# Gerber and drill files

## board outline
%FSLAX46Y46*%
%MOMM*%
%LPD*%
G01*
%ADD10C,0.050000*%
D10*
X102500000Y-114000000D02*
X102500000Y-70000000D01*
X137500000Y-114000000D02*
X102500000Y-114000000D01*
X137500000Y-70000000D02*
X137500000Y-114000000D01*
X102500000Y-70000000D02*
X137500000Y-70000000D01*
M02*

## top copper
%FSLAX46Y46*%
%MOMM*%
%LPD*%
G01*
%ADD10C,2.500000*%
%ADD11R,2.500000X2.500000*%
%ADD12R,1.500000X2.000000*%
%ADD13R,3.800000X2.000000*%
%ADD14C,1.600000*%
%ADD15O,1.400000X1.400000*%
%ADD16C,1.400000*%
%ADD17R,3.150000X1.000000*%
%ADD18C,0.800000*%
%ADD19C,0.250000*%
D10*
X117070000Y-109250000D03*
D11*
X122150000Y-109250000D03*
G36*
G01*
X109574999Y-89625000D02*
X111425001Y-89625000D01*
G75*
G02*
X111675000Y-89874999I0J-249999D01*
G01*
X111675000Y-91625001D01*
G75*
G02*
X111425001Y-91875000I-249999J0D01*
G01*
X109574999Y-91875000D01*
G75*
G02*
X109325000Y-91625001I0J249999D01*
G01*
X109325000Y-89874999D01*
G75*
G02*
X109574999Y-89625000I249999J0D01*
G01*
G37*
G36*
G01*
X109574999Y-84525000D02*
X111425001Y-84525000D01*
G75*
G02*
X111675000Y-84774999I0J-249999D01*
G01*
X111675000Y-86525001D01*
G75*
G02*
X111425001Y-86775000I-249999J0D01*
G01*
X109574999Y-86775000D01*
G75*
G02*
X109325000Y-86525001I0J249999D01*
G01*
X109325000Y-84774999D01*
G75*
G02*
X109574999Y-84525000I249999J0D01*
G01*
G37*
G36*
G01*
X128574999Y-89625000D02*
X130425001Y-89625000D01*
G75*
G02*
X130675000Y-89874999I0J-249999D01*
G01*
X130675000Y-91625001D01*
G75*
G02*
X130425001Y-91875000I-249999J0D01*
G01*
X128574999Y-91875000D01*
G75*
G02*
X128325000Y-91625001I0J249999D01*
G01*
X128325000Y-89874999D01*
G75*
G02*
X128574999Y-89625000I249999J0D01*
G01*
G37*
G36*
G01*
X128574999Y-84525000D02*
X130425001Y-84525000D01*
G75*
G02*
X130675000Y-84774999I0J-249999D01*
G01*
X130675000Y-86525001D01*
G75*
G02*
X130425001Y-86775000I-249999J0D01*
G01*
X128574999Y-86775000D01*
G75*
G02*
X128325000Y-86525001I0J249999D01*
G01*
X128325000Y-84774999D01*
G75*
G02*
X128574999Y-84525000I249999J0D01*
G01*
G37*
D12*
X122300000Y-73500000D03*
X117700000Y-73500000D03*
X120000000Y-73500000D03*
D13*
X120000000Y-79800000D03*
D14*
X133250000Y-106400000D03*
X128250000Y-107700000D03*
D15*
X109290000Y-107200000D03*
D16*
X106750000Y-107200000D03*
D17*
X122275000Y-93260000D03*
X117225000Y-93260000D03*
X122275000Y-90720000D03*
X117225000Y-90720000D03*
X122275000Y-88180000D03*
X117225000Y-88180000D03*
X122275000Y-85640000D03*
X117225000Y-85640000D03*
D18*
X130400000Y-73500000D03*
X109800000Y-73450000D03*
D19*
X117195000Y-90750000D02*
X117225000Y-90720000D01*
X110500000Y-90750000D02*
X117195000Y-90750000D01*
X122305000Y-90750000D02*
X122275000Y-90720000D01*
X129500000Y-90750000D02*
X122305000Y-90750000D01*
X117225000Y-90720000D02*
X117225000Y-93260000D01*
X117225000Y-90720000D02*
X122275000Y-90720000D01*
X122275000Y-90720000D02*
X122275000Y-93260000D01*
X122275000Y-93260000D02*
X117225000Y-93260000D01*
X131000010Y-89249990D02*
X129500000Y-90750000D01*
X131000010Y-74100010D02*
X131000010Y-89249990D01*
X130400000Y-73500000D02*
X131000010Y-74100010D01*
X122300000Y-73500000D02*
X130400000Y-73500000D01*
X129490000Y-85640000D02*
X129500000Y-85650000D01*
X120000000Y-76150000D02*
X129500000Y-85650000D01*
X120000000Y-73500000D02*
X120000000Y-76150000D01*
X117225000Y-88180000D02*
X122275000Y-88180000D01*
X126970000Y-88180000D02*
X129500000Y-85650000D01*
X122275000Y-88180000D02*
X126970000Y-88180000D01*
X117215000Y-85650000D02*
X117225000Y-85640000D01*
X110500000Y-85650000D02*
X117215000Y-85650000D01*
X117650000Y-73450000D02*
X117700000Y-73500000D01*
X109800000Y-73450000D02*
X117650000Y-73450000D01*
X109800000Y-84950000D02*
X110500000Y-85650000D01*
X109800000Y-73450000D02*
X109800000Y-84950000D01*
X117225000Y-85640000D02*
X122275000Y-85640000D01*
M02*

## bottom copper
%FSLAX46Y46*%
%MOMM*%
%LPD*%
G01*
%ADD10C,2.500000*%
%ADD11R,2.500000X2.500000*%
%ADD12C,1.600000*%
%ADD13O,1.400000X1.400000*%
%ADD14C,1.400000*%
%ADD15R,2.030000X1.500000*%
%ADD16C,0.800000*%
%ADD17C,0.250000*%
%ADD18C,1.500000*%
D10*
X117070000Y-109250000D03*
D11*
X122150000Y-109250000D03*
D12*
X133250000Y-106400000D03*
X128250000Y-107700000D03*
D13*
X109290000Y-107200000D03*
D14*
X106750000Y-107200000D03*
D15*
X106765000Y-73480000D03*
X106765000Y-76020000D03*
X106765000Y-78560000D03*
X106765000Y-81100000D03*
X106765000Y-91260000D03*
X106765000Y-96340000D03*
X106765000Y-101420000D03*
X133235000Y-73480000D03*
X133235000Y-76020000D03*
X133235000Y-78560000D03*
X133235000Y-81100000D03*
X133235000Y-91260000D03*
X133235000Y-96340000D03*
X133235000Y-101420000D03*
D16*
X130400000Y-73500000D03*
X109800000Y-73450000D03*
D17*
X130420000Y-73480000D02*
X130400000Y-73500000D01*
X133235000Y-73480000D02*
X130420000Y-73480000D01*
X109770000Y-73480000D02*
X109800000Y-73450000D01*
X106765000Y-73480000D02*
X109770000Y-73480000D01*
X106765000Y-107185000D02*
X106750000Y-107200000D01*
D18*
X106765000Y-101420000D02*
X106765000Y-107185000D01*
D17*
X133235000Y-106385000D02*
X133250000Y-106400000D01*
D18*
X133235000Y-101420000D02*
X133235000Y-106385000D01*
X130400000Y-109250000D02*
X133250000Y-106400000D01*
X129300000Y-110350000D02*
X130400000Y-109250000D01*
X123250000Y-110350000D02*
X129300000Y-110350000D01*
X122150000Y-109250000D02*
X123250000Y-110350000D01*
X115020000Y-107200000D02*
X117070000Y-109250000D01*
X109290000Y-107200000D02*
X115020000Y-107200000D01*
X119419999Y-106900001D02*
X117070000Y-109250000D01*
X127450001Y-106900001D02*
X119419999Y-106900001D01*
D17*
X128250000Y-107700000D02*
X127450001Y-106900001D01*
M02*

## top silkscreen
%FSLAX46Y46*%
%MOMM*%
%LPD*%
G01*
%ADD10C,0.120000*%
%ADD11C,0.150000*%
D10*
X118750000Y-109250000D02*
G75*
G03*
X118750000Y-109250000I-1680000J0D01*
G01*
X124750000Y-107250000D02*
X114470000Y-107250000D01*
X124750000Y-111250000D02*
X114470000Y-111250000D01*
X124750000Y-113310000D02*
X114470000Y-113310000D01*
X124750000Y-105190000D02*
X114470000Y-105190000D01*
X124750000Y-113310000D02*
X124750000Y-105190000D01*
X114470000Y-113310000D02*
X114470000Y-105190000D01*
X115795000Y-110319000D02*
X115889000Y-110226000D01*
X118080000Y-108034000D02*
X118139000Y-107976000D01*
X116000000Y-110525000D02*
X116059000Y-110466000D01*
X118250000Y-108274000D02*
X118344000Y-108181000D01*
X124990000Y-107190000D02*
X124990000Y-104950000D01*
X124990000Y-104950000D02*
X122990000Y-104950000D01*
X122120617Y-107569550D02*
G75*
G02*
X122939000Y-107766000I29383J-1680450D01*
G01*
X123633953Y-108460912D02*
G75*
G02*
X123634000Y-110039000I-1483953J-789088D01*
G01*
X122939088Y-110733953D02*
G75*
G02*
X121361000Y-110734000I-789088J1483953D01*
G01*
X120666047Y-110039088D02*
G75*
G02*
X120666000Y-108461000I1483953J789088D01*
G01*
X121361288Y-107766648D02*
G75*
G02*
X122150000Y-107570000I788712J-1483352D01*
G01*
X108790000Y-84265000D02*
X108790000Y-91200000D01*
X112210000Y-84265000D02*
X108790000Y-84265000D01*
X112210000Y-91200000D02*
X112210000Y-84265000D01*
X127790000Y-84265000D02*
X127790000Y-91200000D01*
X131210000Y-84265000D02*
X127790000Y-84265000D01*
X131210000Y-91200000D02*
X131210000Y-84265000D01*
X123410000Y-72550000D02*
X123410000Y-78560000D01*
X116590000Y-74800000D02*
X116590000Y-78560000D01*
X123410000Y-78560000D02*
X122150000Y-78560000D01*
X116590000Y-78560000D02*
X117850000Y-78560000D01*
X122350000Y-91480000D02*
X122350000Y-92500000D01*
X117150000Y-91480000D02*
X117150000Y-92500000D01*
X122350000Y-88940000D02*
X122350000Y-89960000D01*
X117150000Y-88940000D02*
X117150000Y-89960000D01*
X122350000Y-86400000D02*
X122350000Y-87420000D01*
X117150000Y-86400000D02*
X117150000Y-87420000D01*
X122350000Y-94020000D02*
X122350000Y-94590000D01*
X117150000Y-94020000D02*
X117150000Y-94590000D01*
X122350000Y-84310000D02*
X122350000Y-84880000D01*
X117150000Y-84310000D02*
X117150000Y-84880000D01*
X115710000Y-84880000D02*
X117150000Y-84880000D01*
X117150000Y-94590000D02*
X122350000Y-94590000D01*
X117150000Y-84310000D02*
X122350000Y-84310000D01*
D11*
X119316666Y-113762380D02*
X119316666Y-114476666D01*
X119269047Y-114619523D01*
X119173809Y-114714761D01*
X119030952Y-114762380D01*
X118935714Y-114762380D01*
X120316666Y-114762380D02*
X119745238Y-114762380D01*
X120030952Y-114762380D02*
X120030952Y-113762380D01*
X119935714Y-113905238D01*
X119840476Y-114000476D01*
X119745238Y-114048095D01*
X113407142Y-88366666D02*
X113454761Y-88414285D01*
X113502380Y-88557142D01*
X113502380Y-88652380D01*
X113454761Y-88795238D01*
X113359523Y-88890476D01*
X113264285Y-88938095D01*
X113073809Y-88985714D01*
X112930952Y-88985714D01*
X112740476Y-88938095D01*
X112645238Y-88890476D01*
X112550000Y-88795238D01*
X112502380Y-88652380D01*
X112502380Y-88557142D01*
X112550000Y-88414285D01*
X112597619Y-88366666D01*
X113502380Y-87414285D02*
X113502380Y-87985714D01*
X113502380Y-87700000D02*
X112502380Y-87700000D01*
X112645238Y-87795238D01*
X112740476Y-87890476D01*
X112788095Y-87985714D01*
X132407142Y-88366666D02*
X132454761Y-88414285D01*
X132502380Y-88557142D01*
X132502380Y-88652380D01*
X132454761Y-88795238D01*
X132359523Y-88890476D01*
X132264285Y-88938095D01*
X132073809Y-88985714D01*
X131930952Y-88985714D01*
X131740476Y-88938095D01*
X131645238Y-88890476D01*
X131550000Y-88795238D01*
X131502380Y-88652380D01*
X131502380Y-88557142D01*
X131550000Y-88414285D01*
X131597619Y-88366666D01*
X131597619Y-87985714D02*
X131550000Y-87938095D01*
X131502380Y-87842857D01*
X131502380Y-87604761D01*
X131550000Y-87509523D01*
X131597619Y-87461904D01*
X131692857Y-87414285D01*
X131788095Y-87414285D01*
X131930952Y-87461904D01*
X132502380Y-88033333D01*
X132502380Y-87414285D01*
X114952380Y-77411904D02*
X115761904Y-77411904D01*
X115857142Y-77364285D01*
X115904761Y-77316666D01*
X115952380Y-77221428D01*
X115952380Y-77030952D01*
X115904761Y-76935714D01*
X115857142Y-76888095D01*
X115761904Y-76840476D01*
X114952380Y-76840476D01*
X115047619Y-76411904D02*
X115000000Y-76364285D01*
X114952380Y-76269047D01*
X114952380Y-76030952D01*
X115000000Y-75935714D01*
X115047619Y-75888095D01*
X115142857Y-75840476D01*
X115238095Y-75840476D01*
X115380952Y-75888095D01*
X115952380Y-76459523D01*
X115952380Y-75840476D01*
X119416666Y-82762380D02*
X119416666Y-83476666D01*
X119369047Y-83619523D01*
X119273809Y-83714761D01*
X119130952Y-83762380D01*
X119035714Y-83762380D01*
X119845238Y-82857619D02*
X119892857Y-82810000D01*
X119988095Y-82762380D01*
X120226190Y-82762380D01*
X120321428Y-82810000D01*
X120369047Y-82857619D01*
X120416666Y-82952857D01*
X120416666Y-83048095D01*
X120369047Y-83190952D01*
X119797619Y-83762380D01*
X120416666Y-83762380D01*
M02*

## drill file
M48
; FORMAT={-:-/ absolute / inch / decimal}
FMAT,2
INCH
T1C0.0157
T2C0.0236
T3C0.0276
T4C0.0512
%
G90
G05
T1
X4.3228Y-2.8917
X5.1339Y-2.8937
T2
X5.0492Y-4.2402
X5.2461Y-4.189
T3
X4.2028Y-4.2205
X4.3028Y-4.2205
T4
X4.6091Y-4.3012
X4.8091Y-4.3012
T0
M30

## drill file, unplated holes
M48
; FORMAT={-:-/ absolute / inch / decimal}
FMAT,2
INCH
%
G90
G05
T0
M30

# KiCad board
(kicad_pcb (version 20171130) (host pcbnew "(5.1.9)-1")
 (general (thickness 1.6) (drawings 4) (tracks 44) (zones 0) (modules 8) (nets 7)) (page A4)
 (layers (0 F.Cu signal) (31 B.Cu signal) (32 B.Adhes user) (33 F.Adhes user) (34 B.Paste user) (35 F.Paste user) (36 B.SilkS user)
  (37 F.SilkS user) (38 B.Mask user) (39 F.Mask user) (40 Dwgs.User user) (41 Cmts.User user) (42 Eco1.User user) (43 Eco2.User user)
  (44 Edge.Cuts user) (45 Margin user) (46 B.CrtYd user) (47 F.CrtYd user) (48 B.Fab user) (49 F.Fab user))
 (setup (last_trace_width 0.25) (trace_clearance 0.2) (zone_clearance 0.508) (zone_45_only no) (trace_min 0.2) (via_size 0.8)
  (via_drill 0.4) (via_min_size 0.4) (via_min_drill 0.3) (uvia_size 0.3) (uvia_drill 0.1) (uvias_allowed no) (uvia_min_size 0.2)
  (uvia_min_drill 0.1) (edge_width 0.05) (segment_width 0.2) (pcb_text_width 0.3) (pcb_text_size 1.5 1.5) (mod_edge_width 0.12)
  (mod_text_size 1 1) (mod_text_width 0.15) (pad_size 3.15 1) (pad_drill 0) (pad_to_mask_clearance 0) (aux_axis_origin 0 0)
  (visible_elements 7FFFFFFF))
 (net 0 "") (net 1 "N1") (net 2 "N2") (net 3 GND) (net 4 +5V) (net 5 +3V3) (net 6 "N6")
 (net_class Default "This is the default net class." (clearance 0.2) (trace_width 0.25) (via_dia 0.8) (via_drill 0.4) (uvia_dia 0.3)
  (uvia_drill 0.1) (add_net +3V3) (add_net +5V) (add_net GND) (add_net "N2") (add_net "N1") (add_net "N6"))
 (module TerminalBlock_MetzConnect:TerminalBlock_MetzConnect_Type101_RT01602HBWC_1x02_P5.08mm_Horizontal (layer F.Cu) (at 122.15 109.25 180)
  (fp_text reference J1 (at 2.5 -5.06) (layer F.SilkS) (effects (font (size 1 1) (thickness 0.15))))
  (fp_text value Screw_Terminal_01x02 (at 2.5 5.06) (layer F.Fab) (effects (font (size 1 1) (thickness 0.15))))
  (fp_circle (center 5.08 0) (end 6.76 0) (layer F.SilkS) (width 0.12))
  (fp_line (start -2.6 2) (end 7.68 2) (layer F.SilkS) (width 0.12))
  (fp_line (start -2.6 -2) (end 7.68 -2) (layer F.SilkS) (width 0.12))
  (fp_line (start -2.6 -4.06) (end 7.68 -4.06) (layer F.SilkS) (width 0.12))
  (fp_line (start -2.6 4.06) (end 7.68 4.06) (layer F.SilkS) (width 0.12))
  (fp_line (start -2.6 -4.06) (end -2.6 4.06) (layer F.SilkS) (width 0.12))
  (fp_line (start 7.68 -4.06) (end 7.68 4.06) (layer F.SilkS) (width 0.12))
  (fp_line (start 6.355 -1.069) (end 6.261 -0.976) (layer F.SilkS) (width 0.12))
  (fp_line (start 4.07 1.216) (end 4.011 1.274) (layer F.SilkS) (width 0.12))
  (fp_line (start 6.15 -1.275) (end 6.091 -1.216) (layer F.SilkS) (width 0.12))
  (fp_line (start 3.9 0.976) (end 3.806 1.069) (layer F.SilkS) (width 0.12))
  (fp_line (start -2.84 2.06) (end -2.84 4.3) (layer F.SilkS) (width 0.12))
  (fp_line (start -2.84 4.3) (end -0.84 4.3) (layer F.SilkS) (width 0.12))
  (fp_arc (start 0 0) (end -0.789 1.484) (angle -29) (layer F.SilkS) (width 0.12))
  (fp_arc (start 0 0) (end -1.484 -0.789) (angle -56) (layer F.SilkS) (width 0.12))
  (fp_arc (start 0 0) (end 0.789 -1.484) (angle -56) (layer F.SilkS) (width 0.12))
  (fp_arc (start 0 0) (end 1.484 0.789) (angle -56) (layer F.SilkS) (width 0.12))
  (fp_arc (start 0 0) (end 0 1.68) (angle -28) (layer F.SilkS) (width 0.12))
  (pad 2 thru_hole circle (at 5.08 0 180) (size 2.5 2.5) (drill 1.3) (layers *.Cu *.Mask) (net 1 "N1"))
  (pad 1 thru_hole rect (at 0 0 180) (size 2.5 2.5) (drill 1.3) (layers *.Cu *.Mask) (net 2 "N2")))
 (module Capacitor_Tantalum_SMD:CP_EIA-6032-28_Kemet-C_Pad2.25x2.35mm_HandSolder (layer F.Cu) (at 110.5 88.2 270)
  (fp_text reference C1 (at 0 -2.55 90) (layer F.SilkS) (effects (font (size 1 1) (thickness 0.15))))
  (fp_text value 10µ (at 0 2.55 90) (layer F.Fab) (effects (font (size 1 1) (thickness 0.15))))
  (fp_line (start -3.935 1.71) (end 3 1.71) (layer F.SilkS) (width 0.12))
  (fp_line (start -3.935 -1.71) (end -3.935 1.71) (layer F.SilkS) (width 0.12))
  (fp_line (start 3 -1.71) (end -3.935 -1.71) (layer F.SilkS) (width 0.12))
  (pad 2 smd roundrect (at 2.55 0 270) (size 2.25 2.35) (layers F.Cu F.Paste F.Mask) (roundrect_rratio 0.1111106666666667) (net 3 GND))
  (pad 1 smd roundrect (at -2.55 0 270) (size 2.25 2.35) (layers F.Cu F.Paste F.Mask) (roundrect_rratio 0.1111106666666667) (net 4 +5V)))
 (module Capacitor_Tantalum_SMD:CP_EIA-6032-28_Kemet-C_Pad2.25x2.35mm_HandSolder (layer F.Cu) (at 129.5 88.2 270)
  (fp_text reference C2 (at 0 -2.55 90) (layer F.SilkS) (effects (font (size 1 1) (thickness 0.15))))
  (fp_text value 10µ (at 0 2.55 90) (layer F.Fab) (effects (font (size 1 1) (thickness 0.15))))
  (fp_line (start -3.935 1.71) (end 3 1.71) (layer F.SilkS) (width 0.12))
  (fp_line (start -3.935 -1.71) (end -3.935 1.71) (layer F.SilkS) (width 0.12))
  (fp_line (start 3 -1.71) (end -3.935 -1.71) (layer F.SilkS) (width 0.12))
  (pad 2 smd roundrect (at 2.55 0 270) (size 2.25 2.35) (layers F.Cu F.Paste F.Mask) (roundrect_rratio 0.1111106666666667) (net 3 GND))
  (pad 1 smd roundrect (at -2.55 0 270) (size 2.25 2.35) (layers F.Cu F.Paste F.Mask) (roundrect_rratio 0.1111106666666667) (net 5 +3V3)))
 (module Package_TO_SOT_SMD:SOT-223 (layer F.Cu) (at 120 76.65 270)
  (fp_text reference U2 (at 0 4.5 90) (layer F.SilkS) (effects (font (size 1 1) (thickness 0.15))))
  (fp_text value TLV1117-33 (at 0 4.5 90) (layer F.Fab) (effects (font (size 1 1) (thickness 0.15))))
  (fp_line (start -4.1 -3.41) (end 1.91 -3.41) (layer F.SilkS) (width 0.12))
  (fp_line (start -1.85 3.41) (end 1.91 3.41) (layer F.SilkS) (width 0.12))
  (fp_line (start 1.91 -3.41) (end 1.91 -2.15) (layer F.SilkS) (width 0.12))
  (fp_line (start 1.91 3.41) (end 1.91 2.15) (layer F.SilkS) (width 0.12))
  (pad 1 smd rect (at -3.15 -2.3 270) (size 2 1.5) (layers F.Cu F.Paste F.Mask) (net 3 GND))
  (pad 3 smd rect (at -3.15 2.3 270) (size 2 1.5) (layers F.Cu F.Paste F.Mask) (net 4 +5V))
  (pad 2 smd rect (at -3.15 0 270) (size 2 1.5) (layers F.Cu F.Paste F.Mask) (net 5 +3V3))
  (pad 4 smd rect (at 3.15 0 270) (size 2 3.8) (layers F.Cu F.Paste F.Mask)))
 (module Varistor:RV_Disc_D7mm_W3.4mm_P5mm (layer B.Cu) (at 128.25 107.7)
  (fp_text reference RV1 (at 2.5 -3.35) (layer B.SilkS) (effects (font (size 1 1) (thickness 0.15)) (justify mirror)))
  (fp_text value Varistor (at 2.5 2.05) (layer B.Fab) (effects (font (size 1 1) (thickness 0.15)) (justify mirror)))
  (pad 2 thru_hole circle (at 5 -1.3) (size 1.6 1.6) (drill 0.6) (layers *.Cu *.Mask) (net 2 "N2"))
  (pad 1 thru_hole circle (at 0 0) (size 1.6 1.6) (drill 0.6) (layers *.Cu *.Mask) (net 1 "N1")))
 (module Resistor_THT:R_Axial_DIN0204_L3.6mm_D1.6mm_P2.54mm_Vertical (layer B.Cu) (at 106.75 107.2)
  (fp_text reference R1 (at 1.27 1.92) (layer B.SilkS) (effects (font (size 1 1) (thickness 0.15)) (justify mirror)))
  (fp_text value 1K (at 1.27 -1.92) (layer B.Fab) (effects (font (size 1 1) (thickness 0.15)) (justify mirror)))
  (pad 2 thru_hole oval (at 2.54 0) (size 1.4 1.4) (drill 0.7) (layers *.Cu *.Mask) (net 1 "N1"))
  (pad 1 thru_hole circle (at 0 0) (size 1.4 1.4) (drill 0.7) (layers *.Cu *.Mask) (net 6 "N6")))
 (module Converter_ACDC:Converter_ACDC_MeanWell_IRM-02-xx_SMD (layer B.Cu) (at 120 87.45)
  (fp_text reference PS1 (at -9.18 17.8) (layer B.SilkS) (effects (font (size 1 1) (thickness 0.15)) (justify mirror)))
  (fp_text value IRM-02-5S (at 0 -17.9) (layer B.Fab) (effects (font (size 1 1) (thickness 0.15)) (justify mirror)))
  (pad 12 smd rect (at -13.235 -13.97 90) (size 1.5 2.03) (layers B.Cu B.Paste B.Mask) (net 4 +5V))
  (pad 11 smd rect (at -13.235 -11.43 90) (size 1.5 2.03) (layers B.Cu B.Paste B.Mask))
  (pad 10 smd rect (at -13.235 -8.89 90) (size 1.5 2.03) (layers B.Cu B.Paste B.Mask))
  (pad 9 smd rect (at -13.235 -6.35 90) (size 1.5 2.03) (layers B.Cu B.Paste B.Mask))
  (pad 5 smd rect (at -13.235 3.81 90) (size 1.5 2.03) (layers B.Cu B.Paste B.Mask))
  (pad 3 smd rect (at -13.235 8.89 90) (size 1.5 2.03) (layers B.Cu B.Paste B.Mask))
  (pad 1 smd rect (at -13.235 13.97 90) (size 1.5 2.03) (layers B.Cu B.Paste B.Mask) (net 6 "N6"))
  (pad 13 smd rect (at 13.235 -13.97 90) (size 1.5 2.03) (layers B.Cu B.Paste B.Mask) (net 3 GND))
  (pad 14 smd rect (at 13.235 -11.43 90) (size 1.5 2.03) (layers B.Cu B.Paste B.Mask))
  (pad 15 smd rect (at 13.235 -8.89 90) (size 1.5 2.03) (layers B.Cu B.Paste B.Mask))
  (pad 16 smd rect (at 13.235 -6.35 90) (size 1.5 2.03) (layers B.Cu B.Paste B.Mask))
  (pad 20 smd rect (at 13.235 3.81 90) (size 1.5 2.03) (layers B.Cu B.Paste B.Mask))
  (pad 22 smd rect (at 13.235 8.89 90) (size 1.5 2.03) (layers B.Cu B.Paste B.Mask))
  (pad 24 smd rect (at 13.235 13.97 90) (size 1.5 2.03) (layers B.Cu B.Paste B.Mask) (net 2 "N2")))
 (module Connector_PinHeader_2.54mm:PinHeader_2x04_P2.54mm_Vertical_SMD (layer F.Cu) (at 119.75 89.45)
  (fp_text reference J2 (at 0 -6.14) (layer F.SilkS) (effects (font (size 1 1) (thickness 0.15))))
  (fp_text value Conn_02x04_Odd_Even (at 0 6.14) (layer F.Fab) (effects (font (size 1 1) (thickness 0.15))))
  (fp_line (start 2.6 2.03) (end 2.6 3.05) (layer F.SilkS) (width 0.12))
  (fp_line (start -2.6 2.03) (end -2.6 3.05) (layer F.SilkS) (width 0.12))
  (fp_line (start 2.6 -0.51) (end 2.6 0.51) (layer F.SilkS) (width 0.12))
  (fp_line (start -2.6 -0.51) (end -2.6 0.51) (layer F.SilkS) (width 0.12))
  (fp_line (start 2.6 -3.05) (end 2.6 -2.03) (layer F.SilkS) (width 0.12))
  (fp_line (start -2.6 -3.05) (end -2.6 -2.03) (layer F.SilkS) (width 0.12))
  (fp_line (start 2.6 4.57) (end 2.6 5.14) (layer F.SilkS) (width 0.12))
  (fp_line (start -2.6 4.57) (end -2.6 5.14) (layer F.SilkS) (width 0.12))
  (fp_line (start 2.6 -5.14) (end 2.6 -4.57) (layer F.SilkS) (width 0.12))
  (fp_line (start -2.6 -5.14) (end -2.6 -4.57) (layer F.SilkS) (width 0.12))
  (fp_line (start -4.04 -4.57) (end -2.6 -4.57) (layer F.SilkS) (width 0.12))
  (fp_line (start -2.6 5.14) (end 2.6 5.14) (layer F.SilkS) (width 0.12))
  (fp_line (start -2.6 -5.14) (end 2.6 -5.14) (layer F.SilkS) (width 0.12))
  (pad 8 smd rect (at 2.525 3.81) (size 3.15 1) (layers F.Cu F.Paste F.Mask) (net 3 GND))
  (pad 7 smd rect (at -2.525 3.81) (size 3.15 1) (layers F.Cu F.Paste F.Mask) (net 3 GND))
  (pad 6 smd rect (at 2.525 1.27) (size 3.15 1) (layers F.Cu F.Paste F.Mask) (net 3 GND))
  (pad 5 smd rect (at -2.525 1.27) (size 3.15 1) (layers F.Cu F.Paste F.Mask) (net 3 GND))
  (pad 4 smd rect (at 2.525 -1.27) (size 3.15 1) (layers F.Cu F.Paste F.Mask) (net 5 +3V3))
  (pad 3 smd rect (at -2.525 -1.27) (size 3.15 1) (layers F.Cu F.Paste F.Mask) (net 5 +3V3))
  (pad 2 smd rect (at 2.525 -3.81) (size 3.15 1) (layers F.Cu F.Paste F.Mask) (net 4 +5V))
  (pad 1 smd rect (at -2.525 -3.81) (size 3.15 1) (layers F.Cu F.Paste F.Mask) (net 4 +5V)))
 (gr_line (start 102.5 114) (end 102.5 70) (layer Edge.Cuts) (width 0.05))
 (gr_line (start 137.5 114) (end 102.5 114) (layer Edge.Cuts) (width 0.05))
 (gr_line (start 137.5 70) (end 137.5 114) (layer Edge.Cuts) (width 0.05))
 (gr_line (start 102.5 70) (end 137.5 70) (layer Edge.Cuts) (width 0.05))
 (via (at 130.4 73.5) (size 0.8) (drill 0.4) (layers F.Cu B.Cu) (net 3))
 (segment (start 117.195 90.75) (end 117.225 90.72) (width 0.25) (layer F.Cu) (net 3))
 (segment (start 110.5 90.75) (end 117.195 90.75) (width 0.25) (layer F.Cu) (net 3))
 (segment (start 122.305 90.75) (end 122.275 90.72) (width 0.25) (layer F.Cu) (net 3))
 (segment (start 129.5 90.75) (end 122.305 90.75) (width 0.25) (layer F.Cu) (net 3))
 (segment (start 117.225 90.72) (end 117.225 93.26) (width 0.25) (layer F.Cu) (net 3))
 (segment (start 117.225 90.72) (end 122.275 90.72) (width 0.25) (layer F.Cu) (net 3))
 (segment (start 122.275 90.72) (end 122.275 93.26) (width 0.25) (layer F.Cu) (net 3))
 (segment (start 122.275 93.26) (end 117.225 93.26) (width 0.25) (layer F.Cu) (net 3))
 (segment (start 130.42 73.48) (end 130.4 73.5) (width 0.25) (layer B.Cu) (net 3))
 (segment (start 133.235 73.48) (end 130.42 73.48) (width 0.25) (layer B.Cu) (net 3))
 (segment (start 131.00001 89.24999) (end 129.5 90.75) (width 0.25) (layer F.Cu) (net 3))
 (segment (start 131.00001 74.10001) (end 131.00001 89.24999) (width 0.25) (layer F.Cu) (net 3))
 (segment (start 130.4 73.5) (end 131.00001 74.10001) (width 0.25) (layer F.Cu) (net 3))
 (segment (start 122.3 73.5) (end 130.4 73.5) (width 0.25) (layer F.Cu) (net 3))
 (segment (start 129.49 85.64) (end 129.5 85.65) (width 0.25) (layer F.Cu) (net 5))
 (segment (start 120 76.15) (end 129.5 85.65) (width 0.25) (layer F.Cu) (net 5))
 (segment (start 120 73.5) (end 120 76.15) (width 0.25) (layer F.Cu) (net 5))
 (segment (start 117.225 88.18) (end 122.275 88.18) (width 0.25) (layer F.Cu) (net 5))
 (segment (start 126.97 88.18) (end 129.5 85.65) (width 0.25) (layer F.Cu) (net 5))
 (segment (start 122.275 88.18) (end 126.97 88.18) (width 0.25) (layer F.Cu) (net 5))
 (via (at 109.8 73.45) (size 0.8) (drill 0.4) (layers F.Cu B.Cu) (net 4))
 (segment (start 117.215 85.65) (end 117.225 85.64) (width 0.25) (layer F.Cu) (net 4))
 (segment (start 110.5 85.65) (end 117.215 85.65) (width 0.25) (layer F.Cu) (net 4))
 (segment (start 109.77 73.48) (end 109.8 73.45) (width 0.25) (layer B.Cu) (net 4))
 (segment (start 106.765 73.48) (end 109.77 73.48) (width 0.25) (layer B.Cu) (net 4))
 (segment (start 117.65 73.45) (end 117.7 73.5) (width 0.25) (layer F.Cu) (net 4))
 (segment (start 109.8 73.45) (end 117.65 73.45) (width 0.25) (layer F.Cu) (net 4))
 (segment (start 109.8 84.95) (end 110.5 85.65) (width 0.25) (layer F.Cu) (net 4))
 (segment (start 109.8 73.45) (end 109.8 84.95) (width 0.25) (layer F.Cu) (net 4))
 (segment (start 117.225 85.64) (end 122.275 85.64) (width 0.25) (layer F.Cu) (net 4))
 (segment (start 106.765 107.185) (end 106.75 107.2) (width 0.25) (layer B.Cu) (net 6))
 (segment (start 106.765 101.42) (end 106.765 107.185) (width 1.5) (layer B.Cu) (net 6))
 (segment (start 133.235 106.385) (end 133.25 106.4) (width 0.25) (layer B.Cu) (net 2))
 (segment (start 133.235 101.42) (end 133.235 106.385) (width 1.5) (layer B.Cu) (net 2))
 (segment (start 130.4 109.25) (end 133.25 106.4) (width 1.5) (layer B.Cu) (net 2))
 (segment (start 129.3 110.35) (end 130.4 109.25) (width 1.5) (layer B.Cu) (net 2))
 (segment (start 123.25 110.35) (end 129.3 110.35) (width 1.5) (layer B.Cu) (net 2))
 (segment (start 122.15 109.25) (end 123.25 110.35) (width 1.5) (layer B.Cu) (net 2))
 (segment (start 115.02 107.2) (end 117.07 109.25) (width 1.5) (layer B.Cu) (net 1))
 (segment (start 109.29 107.2) (end 115.02 107.2) (width 1.5) (layer B.Cu) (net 1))
 (segment (start 119.419999 106.900001) (end 117.07 109.25) (width 1.5) (layer B.Cu) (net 1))
 (segment (start 127.450001 106.900001) (end 119.419999 106.900001) (width 1.5) (layer B.Cu) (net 1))
 (segment (start 128.25 107.7) (end 127.450001 106.900001) (width 0.25) (layer B.Cu) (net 1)))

